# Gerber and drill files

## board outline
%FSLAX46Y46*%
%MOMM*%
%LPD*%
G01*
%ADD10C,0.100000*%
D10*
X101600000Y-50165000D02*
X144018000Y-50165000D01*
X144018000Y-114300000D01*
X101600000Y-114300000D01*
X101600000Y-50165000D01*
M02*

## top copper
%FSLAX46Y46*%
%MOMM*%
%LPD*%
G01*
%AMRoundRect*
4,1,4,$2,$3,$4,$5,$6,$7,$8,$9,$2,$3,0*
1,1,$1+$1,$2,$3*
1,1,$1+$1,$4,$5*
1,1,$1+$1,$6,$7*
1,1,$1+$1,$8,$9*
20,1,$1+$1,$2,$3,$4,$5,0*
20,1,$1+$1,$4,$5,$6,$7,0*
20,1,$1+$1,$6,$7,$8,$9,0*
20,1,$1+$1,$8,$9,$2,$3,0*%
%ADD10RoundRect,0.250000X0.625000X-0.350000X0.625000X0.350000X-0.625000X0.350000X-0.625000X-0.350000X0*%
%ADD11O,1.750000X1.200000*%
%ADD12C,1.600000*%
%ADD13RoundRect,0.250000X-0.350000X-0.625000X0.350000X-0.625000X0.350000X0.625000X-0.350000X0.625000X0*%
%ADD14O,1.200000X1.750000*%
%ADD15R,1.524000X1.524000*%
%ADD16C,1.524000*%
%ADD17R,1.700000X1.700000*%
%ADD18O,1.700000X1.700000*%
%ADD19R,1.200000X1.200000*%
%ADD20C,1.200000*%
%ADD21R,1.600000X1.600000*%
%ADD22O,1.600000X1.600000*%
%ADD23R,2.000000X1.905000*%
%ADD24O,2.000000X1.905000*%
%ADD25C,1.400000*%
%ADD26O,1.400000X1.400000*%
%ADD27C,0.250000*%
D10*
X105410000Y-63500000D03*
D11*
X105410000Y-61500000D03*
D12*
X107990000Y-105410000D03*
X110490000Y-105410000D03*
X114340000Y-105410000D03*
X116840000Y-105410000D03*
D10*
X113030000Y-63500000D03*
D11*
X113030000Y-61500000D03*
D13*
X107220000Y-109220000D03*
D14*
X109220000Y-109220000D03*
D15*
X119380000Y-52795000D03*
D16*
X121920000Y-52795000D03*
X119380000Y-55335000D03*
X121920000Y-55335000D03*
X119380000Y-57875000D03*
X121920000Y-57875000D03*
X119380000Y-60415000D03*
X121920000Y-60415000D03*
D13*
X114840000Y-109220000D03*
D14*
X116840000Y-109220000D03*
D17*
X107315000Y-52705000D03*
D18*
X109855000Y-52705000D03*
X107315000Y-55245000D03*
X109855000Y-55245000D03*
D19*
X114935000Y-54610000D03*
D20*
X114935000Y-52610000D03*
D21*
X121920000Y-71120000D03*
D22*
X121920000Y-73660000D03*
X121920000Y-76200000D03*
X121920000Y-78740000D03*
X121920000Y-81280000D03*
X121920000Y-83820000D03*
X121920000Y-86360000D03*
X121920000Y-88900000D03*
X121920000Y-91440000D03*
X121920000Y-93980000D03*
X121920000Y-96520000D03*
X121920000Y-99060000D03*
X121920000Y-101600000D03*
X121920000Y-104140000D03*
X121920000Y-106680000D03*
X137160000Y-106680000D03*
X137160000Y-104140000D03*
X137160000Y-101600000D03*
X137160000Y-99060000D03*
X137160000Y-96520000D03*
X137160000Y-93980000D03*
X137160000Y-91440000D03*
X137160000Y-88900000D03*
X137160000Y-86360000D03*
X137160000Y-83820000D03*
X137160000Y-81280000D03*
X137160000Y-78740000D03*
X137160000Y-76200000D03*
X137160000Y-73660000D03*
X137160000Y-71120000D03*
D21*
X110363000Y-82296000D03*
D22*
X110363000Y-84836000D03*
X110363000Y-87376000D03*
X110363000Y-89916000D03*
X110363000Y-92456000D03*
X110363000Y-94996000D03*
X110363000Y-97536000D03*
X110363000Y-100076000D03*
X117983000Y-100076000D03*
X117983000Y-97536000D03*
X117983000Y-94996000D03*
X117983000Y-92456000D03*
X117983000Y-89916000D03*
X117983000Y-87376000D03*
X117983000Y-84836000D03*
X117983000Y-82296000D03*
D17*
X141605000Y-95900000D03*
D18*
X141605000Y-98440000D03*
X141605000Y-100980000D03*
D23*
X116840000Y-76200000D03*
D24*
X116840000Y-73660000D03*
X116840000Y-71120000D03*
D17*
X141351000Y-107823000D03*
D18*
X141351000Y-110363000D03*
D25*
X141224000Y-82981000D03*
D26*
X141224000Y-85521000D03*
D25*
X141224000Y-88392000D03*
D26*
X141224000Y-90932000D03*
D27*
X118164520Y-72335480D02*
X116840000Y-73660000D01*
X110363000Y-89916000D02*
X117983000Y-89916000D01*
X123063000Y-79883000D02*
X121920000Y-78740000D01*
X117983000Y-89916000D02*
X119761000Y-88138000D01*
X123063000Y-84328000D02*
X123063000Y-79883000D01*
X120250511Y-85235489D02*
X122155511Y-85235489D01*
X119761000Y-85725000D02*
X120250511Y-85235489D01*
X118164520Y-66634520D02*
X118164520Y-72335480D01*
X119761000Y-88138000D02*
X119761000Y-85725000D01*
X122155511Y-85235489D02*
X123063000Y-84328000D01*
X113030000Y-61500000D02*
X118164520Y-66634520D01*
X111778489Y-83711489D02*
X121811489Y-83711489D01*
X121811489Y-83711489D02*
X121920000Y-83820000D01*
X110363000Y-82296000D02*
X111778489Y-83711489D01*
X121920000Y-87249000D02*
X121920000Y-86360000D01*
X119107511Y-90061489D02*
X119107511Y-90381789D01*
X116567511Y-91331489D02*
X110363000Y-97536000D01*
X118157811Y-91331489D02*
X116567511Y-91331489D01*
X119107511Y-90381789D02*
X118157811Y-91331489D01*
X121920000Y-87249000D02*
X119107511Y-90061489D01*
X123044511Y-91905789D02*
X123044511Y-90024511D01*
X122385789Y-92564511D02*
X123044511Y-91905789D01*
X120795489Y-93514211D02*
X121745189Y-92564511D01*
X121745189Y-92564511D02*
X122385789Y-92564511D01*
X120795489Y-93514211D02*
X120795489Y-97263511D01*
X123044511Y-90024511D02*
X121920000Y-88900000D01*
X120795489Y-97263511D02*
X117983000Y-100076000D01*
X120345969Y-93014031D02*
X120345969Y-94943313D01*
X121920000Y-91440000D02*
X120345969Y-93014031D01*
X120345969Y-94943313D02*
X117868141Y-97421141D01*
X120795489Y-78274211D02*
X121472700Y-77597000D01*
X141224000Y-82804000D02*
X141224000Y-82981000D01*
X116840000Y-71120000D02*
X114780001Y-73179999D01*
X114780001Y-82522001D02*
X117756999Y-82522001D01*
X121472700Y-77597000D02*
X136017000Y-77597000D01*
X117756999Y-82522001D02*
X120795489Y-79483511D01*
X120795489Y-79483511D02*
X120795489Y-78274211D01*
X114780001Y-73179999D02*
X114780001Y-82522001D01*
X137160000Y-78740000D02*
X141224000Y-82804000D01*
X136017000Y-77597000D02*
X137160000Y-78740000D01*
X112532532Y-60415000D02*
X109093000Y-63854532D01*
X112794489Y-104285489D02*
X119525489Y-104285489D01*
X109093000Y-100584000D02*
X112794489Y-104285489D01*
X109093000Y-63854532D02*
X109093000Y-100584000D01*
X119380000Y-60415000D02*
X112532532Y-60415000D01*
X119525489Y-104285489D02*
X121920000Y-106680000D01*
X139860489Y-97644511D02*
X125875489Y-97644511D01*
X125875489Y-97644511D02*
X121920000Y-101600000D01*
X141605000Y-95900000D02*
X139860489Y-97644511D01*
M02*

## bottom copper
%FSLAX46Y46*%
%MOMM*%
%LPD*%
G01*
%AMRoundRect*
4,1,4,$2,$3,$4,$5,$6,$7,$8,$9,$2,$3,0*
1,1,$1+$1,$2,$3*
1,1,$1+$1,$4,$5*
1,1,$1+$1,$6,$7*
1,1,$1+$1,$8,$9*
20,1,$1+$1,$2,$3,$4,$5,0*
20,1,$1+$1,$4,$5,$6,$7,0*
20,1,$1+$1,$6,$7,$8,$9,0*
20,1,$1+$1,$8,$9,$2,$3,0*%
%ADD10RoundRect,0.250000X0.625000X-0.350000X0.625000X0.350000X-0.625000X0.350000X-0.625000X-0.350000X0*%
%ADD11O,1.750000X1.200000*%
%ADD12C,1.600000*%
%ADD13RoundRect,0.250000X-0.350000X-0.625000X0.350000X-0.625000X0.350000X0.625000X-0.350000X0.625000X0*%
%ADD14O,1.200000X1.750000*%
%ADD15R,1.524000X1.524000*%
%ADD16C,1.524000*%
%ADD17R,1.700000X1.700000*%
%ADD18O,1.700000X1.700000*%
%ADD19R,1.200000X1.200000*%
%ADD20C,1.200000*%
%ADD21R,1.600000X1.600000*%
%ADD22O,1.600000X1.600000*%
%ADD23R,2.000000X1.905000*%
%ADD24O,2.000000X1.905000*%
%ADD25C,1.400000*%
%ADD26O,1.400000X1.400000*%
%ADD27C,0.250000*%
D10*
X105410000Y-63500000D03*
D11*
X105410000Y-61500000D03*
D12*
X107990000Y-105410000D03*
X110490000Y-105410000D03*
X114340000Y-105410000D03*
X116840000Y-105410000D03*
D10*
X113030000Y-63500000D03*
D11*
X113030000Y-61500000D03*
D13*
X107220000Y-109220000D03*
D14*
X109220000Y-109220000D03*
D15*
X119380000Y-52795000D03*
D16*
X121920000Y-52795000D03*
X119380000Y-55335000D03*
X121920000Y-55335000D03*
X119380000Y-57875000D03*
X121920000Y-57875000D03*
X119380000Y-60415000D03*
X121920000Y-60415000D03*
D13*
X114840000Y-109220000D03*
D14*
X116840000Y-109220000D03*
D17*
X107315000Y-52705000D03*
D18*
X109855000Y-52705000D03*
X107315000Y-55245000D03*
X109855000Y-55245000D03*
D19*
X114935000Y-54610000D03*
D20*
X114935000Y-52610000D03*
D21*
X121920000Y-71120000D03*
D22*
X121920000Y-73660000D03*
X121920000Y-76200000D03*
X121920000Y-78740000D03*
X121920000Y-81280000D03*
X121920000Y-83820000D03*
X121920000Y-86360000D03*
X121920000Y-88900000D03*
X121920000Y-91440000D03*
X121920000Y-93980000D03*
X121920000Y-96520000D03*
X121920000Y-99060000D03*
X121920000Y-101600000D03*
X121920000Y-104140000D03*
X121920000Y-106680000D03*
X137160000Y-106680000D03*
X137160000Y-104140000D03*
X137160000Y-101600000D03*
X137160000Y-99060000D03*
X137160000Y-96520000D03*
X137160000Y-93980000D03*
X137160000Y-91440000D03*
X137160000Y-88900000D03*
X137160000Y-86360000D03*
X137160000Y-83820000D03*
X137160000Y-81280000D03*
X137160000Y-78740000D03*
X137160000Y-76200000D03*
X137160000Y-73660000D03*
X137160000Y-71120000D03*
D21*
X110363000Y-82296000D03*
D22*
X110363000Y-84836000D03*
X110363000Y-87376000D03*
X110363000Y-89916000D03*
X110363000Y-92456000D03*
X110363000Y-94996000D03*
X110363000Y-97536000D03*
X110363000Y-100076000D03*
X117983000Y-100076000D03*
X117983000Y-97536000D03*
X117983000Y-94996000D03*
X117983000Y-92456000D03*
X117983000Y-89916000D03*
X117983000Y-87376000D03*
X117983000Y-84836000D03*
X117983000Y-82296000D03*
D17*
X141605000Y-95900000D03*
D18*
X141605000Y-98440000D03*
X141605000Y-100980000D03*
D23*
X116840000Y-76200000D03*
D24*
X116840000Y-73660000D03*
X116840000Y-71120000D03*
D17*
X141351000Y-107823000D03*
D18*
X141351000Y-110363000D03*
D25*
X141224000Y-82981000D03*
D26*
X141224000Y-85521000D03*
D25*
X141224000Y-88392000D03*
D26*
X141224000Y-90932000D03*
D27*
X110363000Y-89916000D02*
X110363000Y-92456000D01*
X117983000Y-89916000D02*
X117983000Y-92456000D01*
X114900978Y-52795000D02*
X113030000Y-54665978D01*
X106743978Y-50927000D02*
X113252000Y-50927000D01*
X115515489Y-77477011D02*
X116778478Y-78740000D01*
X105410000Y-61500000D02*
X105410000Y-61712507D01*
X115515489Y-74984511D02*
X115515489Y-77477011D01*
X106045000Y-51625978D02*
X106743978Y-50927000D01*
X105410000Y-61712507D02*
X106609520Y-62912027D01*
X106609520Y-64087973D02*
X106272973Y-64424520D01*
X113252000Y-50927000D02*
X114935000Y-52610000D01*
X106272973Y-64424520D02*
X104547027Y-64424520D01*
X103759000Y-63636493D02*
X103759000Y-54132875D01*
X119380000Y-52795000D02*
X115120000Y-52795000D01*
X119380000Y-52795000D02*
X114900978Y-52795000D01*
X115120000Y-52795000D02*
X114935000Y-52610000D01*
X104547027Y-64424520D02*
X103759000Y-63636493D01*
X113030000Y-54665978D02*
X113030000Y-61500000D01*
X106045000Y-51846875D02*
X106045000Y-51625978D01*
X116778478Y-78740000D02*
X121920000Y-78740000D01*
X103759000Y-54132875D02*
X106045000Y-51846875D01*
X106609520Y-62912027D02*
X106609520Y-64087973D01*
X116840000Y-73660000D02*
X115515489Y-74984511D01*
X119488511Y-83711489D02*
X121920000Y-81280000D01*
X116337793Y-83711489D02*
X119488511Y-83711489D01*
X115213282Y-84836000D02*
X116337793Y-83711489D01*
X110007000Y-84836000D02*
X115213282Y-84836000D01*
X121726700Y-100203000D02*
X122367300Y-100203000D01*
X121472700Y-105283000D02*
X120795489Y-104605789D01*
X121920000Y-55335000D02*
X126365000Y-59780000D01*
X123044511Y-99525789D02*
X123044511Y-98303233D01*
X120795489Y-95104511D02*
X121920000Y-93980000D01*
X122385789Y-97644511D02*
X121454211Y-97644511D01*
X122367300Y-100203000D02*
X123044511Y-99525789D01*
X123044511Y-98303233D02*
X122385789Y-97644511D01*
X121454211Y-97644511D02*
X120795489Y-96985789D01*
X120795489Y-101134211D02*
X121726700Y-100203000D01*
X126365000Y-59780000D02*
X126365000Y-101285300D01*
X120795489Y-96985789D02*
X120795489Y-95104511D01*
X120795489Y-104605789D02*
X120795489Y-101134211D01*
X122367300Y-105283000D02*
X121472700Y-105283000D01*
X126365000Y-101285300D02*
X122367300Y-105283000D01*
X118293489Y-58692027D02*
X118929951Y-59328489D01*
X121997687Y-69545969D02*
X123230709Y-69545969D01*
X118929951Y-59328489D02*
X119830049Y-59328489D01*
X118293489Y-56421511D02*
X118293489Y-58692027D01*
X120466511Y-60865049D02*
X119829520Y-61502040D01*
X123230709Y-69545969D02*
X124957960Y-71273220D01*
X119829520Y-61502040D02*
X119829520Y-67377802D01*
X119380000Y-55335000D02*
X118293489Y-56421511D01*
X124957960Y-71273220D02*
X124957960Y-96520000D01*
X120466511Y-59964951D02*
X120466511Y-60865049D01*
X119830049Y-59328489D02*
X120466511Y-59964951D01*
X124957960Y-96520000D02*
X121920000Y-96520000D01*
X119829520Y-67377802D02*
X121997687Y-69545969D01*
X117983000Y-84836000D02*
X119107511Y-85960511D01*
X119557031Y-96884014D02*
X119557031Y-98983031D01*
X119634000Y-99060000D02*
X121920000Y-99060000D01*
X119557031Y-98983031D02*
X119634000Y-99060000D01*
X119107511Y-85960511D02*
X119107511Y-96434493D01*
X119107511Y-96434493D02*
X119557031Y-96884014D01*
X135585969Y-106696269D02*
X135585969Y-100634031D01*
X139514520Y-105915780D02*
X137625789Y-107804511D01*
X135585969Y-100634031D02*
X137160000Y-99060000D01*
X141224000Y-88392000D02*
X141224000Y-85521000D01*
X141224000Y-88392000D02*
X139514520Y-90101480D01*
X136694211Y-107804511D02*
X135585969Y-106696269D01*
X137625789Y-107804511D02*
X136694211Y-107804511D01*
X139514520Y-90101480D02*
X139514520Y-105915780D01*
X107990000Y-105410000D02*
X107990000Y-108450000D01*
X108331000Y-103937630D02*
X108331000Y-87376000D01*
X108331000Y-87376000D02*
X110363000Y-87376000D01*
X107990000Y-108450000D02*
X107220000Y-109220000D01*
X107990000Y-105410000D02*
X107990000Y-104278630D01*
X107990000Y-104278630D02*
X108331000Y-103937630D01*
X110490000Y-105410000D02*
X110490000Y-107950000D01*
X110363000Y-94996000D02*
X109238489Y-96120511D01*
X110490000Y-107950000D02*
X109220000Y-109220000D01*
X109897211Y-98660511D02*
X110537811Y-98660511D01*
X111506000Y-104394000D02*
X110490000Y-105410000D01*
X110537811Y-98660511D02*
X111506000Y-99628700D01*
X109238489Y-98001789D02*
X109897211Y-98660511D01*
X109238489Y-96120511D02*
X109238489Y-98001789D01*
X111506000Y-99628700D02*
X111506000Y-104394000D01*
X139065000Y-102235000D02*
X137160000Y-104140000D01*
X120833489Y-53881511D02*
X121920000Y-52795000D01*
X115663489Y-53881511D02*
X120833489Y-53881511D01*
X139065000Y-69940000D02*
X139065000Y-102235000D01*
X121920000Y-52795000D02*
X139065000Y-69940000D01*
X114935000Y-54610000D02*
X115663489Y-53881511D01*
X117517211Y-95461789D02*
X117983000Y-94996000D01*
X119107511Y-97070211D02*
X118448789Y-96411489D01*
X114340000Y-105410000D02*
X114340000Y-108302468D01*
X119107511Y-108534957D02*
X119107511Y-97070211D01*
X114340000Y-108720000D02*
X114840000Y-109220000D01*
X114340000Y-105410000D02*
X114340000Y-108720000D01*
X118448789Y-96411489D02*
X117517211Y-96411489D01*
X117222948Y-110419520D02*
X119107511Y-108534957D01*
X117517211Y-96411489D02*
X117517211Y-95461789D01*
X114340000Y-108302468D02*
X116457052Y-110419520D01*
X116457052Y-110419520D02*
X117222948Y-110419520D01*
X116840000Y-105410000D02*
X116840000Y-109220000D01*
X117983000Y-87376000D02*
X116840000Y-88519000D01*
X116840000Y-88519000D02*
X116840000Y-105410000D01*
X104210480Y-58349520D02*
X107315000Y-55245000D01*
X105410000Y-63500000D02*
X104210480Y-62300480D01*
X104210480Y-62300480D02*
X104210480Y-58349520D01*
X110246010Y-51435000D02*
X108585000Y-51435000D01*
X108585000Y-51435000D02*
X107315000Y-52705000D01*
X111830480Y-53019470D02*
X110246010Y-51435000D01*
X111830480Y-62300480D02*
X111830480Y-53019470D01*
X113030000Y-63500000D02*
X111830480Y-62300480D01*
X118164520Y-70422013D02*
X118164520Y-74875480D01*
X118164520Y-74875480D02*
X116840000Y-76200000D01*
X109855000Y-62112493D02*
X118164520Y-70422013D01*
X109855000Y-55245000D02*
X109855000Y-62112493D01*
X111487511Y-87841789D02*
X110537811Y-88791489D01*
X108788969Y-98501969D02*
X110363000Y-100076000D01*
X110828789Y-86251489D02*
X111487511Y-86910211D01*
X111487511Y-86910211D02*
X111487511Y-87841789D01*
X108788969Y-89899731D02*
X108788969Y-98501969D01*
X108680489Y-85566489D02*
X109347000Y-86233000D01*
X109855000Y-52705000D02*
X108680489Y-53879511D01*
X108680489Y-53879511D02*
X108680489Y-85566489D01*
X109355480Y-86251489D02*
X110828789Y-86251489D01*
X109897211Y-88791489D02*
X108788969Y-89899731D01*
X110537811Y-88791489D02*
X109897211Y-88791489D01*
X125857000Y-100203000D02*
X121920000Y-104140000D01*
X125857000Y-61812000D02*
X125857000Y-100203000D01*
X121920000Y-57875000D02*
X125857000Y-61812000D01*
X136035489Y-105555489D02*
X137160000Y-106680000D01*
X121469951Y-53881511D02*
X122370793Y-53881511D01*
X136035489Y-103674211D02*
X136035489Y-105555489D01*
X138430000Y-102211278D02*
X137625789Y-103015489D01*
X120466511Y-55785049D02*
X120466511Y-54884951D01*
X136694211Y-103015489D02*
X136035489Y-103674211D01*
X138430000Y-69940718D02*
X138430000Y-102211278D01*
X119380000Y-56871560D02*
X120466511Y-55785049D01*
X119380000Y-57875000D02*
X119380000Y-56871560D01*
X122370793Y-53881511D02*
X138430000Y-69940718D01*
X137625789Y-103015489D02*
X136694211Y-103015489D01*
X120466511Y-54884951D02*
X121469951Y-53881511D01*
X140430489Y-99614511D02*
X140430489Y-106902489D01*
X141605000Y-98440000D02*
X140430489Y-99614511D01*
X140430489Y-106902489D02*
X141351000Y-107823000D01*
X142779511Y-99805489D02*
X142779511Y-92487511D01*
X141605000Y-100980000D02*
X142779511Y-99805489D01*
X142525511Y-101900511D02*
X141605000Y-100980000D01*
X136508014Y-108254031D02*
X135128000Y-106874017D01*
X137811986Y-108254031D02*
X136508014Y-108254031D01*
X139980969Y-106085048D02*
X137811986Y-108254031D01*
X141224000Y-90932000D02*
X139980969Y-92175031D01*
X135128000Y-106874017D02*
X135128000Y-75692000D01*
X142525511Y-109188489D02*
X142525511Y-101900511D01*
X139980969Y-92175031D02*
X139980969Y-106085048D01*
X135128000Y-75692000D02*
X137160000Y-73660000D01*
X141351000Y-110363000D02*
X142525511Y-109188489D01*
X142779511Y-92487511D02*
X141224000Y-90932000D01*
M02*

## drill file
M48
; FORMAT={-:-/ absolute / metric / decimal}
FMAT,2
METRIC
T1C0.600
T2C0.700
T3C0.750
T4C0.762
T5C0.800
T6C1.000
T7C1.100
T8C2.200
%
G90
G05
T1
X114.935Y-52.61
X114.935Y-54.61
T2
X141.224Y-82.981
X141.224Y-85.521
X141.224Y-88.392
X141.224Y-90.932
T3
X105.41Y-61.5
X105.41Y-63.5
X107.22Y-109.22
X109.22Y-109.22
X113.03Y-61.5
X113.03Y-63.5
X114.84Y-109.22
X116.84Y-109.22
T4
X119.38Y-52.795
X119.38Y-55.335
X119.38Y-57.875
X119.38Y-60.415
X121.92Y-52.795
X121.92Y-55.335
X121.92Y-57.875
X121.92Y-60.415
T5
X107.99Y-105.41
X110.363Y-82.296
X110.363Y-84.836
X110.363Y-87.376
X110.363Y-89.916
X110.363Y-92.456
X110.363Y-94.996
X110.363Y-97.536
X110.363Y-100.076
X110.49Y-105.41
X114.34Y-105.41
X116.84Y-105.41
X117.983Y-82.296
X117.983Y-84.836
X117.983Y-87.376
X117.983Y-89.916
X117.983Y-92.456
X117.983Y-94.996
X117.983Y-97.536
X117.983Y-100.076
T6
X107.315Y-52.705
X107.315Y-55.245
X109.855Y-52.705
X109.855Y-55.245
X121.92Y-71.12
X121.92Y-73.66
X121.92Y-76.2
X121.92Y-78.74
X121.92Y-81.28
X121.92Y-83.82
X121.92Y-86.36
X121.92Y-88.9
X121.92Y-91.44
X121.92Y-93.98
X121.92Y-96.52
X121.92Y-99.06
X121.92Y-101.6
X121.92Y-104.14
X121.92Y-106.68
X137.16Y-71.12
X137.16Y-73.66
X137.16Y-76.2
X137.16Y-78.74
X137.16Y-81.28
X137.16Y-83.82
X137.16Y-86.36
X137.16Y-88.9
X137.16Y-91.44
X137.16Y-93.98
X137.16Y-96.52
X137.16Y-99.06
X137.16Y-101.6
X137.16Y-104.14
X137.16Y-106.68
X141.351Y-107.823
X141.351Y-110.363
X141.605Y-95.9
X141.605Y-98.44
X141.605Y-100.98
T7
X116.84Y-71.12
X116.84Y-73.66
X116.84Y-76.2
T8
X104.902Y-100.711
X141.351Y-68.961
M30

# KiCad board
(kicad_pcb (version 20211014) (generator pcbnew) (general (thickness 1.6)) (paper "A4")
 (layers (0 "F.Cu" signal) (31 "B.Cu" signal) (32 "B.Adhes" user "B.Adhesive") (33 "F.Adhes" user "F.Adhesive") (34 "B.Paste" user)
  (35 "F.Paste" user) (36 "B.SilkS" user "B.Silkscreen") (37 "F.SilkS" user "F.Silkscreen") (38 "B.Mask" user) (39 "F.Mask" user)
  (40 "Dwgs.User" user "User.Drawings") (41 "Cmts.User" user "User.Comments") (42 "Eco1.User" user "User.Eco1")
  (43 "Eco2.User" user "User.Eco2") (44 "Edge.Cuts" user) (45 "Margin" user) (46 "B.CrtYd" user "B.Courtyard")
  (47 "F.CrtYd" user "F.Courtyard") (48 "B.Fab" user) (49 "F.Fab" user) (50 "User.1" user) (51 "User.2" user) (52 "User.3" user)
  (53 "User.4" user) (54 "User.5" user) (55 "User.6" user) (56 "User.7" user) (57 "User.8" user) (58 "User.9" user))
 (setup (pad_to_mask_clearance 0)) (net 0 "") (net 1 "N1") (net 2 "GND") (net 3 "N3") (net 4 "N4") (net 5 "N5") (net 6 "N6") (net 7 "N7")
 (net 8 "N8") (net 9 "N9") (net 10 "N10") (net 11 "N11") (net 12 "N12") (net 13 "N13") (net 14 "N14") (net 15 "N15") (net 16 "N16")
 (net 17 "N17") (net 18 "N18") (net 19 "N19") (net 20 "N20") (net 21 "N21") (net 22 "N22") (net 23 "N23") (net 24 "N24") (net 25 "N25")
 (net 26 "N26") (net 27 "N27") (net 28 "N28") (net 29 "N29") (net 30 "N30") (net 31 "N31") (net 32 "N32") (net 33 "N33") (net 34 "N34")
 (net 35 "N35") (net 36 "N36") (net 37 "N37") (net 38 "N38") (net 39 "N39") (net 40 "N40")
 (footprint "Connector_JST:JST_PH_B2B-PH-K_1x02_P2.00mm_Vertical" (layer "F.Cu") (at 105.41 63.5 90)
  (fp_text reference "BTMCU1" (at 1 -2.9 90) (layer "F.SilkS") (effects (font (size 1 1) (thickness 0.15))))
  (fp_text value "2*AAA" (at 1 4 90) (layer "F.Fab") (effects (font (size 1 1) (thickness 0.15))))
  (pad "1" thru_hole roundrect (at 0 0 90) (size 1.2 1.75) (drill 0.75) (layers *.Cu *.Mask) (roundrect_rratio 0.2083333333) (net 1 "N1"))
  (pad "2" thru_hole oval (at 2 0 90) (size 1.2 1.75) (drill 0.75) (layers *.Cu *.Mask) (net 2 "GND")))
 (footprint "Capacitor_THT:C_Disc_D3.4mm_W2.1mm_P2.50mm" (layer "F.Cu") (at 107.99 105.41)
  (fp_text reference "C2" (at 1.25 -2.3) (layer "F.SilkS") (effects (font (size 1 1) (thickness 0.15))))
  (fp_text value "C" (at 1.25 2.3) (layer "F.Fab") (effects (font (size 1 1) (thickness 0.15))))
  (pad "1" thru_hole circle (at 0 0) (size 1.6 1.6) (drill 0.8) (layers *.Cu *.Mask) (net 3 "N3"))
  (pad "2" thru_hole circle (at 2.5 0) (size 1.6 1.6) (drill 0.8) (layers *.Cu *.Mask) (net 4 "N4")))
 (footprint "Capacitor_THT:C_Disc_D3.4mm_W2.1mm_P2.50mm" (layer "F.Cu") (at 114.34 105.41)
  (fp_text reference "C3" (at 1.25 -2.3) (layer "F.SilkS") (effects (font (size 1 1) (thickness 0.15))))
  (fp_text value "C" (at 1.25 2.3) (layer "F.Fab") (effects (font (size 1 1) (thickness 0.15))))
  (pad "1" thru_hole circle (at 0 0) (size 1.6 1.6) (drill 0.8) (layers *.Cu *.Mask) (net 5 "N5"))
  (pad "2" thru_hole circle (at 2.5 0) (size 1.6 1.6) (drill 0.8) (layers *.Cu *.Mask) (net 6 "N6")))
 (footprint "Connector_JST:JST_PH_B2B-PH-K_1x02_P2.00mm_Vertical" (layer "F.Cu") (at 113.03 63.5 90)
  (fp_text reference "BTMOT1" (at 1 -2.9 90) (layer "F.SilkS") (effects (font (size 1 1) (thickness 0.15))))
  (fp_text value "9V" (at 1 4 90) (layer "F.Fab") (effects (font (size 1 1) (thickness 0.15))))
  (pad "1" thru_hole roundrect (at 0 0 90) (size 1.2 1.75) (drill 0.75) (layers *.Cu *.Mask) (roundrect_rratio 0.2083333333) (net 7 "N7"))
  (pad "2" thru_hole oval (at 2 0 90) (size 1.2 1.75) (drill 0.75) (layers *.Cu *.Mask) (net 2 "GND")))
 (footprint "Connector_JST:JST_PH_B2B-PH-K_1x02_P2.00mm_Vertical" (layer "F.Cu") (at 107.22 109.22)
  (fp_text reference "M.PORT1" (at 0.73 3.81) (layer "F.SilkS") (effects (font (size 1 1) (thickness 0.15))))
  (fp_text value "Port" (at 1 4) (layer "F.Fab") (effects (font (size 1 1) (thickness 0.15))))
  (pad "1" thru_hole roundrect (at 0 0) (size 1.2 1.75) (drill 0.75) (layers *.Cu *.Mask) (roundrect_rratio 0.2083333333) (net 3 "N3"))
  (pad "2" thru_hole oval (at 2 0) (size 1.2 1.75) (drill 0.75) (layers *.Cu *.Mask) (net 4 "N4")))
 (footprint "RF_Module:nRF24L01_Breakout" (layer "F.Cu") (at 119.38 52.795)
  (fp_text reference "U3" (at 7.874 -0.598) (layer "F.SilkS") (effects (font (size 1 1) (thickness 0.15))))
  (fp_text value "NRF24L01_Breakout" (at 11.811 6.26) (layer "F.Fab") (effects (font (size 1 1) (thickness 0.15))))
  (pad "1" thru_hole rect (at 0 0) (size 1.524 1.524) (drill 0.762) (layers *.Cu *.Mask) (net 2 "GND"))
  (pad "2" thru_hole circle (at 2.54 0) (size 1.524 1.524) (drill 0.762) (layers *.Cu *.Mask) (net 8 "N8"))
  (pad "3" thru_hole circle (at 0 2.54) (size 1.524 1.524) (drill 0.762) (layers *.Cu *.Mask) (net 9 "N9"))
  (pad "4" thru_hole circle (at 2.54 2.54) (size 1.524 1.524) (drill 0.762) (layers *.Cu *.Mask) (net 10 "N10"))
  (pad "5" thru_hole circle (at 0 5.08) (size 1.524 1.524) (drill 0.762) (layers *.Cu *.Mask) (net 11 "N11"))
  (pad "6" thru_hole circle (at 2.54 5.08) (size 1.524 1.524) (drill 0.762) (layers *.Cu *.Mask) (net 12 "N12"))
  (pad "7" thru_hole circle (at 0 7.62) (size 1.524 1.524) (drill 0.762) (layers *.Cu *.Mask) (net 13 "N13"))
  (pad "8" thru_hole circle (at 2.54 7.62) (size 1.524 1.524) (drill 0.762) (layers *.Cu *.Mask) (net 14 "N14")))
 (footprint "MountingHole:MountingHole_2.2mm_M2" (layer "F.Cu") (at 104.902 100.711)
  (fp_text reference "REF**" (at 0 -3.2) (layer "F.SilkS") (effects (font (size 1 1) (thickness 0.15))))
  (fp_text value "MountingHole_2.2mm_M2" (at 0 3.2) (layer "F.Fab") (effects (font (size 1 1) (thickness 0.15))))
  (pad "" np_thru_hole circle (at 0 0) (size 2.2 2.2) (drill 2.2) (layers *.Cu *.Mask)))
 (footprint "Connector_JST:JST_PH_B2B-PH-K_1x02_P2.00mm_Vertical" (layer "F.Cu") (at 114.84 109.22)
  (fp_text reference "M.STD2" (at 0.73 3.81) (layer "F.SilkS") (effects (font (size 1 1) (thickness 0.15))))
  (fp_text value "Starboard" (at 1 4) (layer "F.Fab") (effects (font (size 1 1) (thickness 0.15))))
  (pad "1" thru_hole roundrect (at 0 0) (size 1.2 1.75) (drill 0.75) (layers *.Cu *.Mask) (roundrect_rratio 0.2083333333) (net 5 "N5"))
  (pad "2" thru_hole oval (at 2 0) (size 1.2 1.75) (drill 0.75) (layers *.Cu *.Mask) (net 6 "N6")))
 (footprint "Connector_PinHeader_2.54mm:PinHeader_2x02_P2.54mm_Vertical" (layer "F.Cu") (at 107.315 52.705)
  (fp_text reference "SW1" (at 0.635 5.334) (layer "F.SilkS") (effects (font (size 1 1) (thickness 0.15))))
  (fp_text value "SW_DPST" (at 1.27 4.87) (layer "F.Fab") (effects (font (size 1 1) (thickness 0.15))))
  (pad "1" thru_hole rect (at 0 0) (size 1.7 1.7) (drill 1) (layers *.Cu *.Mask) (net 7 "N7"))
  (pad "2" thru_hole oval (at 2.54 0) (size 1.7 1.7) (drill 1) (layers *.Cu *.Mask) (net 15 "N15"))
  (pad "3" thru_hole oval (at 0 2.54) (size 1.7 1.7) (drill 1) (layers *.Cu *.Mask) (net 1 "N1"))
  (pad "4" thru_hole oval (at 2.54 2.54) (size 1.7 1.7) (drill 1) (layers *.Cu *.Mask) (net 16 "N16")))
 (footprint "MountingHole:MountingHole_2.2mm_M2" (layer "F.Cu") (at 141.351 68.961)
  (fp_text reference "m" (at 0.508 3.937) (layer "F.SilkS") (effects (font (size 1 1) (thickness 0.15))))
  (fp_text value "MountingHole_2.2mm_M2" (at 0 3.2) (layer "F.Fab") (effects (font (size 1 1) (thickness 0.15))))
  (pad "" np_thru_hole circle (at 0 0) (size 2.2 2.2) (drill 2.2) (layers *.Cu *.Mask)))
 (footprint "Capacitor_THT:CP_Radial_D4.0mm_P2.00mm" (layer "F.Cu") (at 114.935 54.61 90)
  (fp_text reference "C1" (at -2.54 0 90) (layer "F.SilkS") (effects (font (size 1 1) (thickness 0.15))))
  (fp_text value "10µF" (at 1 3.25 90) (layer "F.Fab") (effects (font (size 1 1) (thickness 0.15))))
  (pad "1" thru_hole rect (at 0 0 90) (size 1.2 1.2) (drill 0.6) (layers *.Cu *.Mask) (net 8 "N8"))
  (pad "2" thru_hole circle (at 2 0 90) (size 1.2 1.2) (drill 0.6) (layers *.Cu *.Mask) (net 2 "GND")))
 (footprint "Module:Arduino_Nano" (layer "F.Cu") (at 121.92 71.12)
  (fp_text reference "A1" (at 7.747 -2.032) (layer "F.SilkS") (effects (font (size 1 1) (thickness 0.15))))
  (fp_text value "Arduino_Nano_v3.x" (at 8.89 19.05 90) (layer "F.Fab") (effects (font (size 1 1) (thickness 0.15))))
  (pad "1" thru_hole rect (at 0 0) (size 1.6 1.6) (drill 1) (layers *.Cu *.Mask) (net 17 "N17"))
  (pad "2" thru_hole oval (at 0 2.54) (size 1.6 1.6) (drill 1) (layers *.Cu *.Mask) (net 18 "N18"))
  (pad "3" thru_hole oval (at 0 5.08) (size 1.6 1.6) (drill 1) (layers *.Cu *.Mask) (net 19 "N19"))
  (pad "4" thru_hole oval (at 0 7.62) (size 1.6 1.6) (drill 1) (layers *.Cu *.Mask) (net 2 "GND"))
  (pad "5" thru_hole oval (at 0 10.16) (size 1.6 1.6) (drill 1) (layers *.Cu *.Mask) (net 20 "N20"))
  (pad "6" thru_hole oval (at 0 12.7) (size 1.6 1.6) (drill 1) (layers *.Cu *.Mask) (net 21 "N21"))
  (pad "7" thru_hole oval (at 0 15.24) (size 1.6 1.6) (drill 1) (layers *.Cu *.Mask) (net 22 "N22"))
  (pad "8" thru_hole oval (at 0 17.78) (size 1.6 1.6) (drill 1) (layers *.Cu *.Mask) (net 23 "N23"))
  (pad "9" thru_hole oval (at 0 20.32) (size 1.6 1.6) (drill 1) (layers *.Cu *.Mask) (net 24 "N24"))
  (pad "10" thru_hole oval (at 0 22.86) (size 1.6 1.6) (drill 1) (layers *.Cu *.Mask) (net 10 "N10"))
  (pad "11" thru_hole oval (at 0 25.4) (size 1.6 1.6) (drill 1) (layers *.Cu *.Mask) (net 9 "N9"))
  (pad "12" thru_hole oval (at 0 27.94) (size 1.6 1.6) (drill 1) (layers *.Cu *.Mask) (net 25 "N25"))
  (pad "13" thru_hole oval (at 0 30.48) (size 1.6 1.6) (drill 1) (layers *.Cu *.Mask) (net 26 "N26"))
  (pad "14" thru_hole oval (at 0 33.02) (size 1.6 1.6) (drill 1) (layers *.Cu *.Mask) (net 12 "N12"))
  (pad "15" thru_hole oval (at 0 35.56) (size 1.6 1.6) (drill 1) (layers *.Cu *.Mask) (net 13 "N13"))
  (pad "16" thru_hole oval (at 15.24 35.56) (size 1.6 1.6) (drill 1) (layers *.Cu *.Mask) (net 11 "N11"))
  (pad "17" thru_hole oval (at 15.24 33.02) (size 1.6 1.6) (drill 1) (layers *.Cu *.Mask) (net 8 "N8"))
  (pad "18" thru_hole oval (at 15.24 30.48) (size 1.6 1.6) (drill 1) (layers *.Cu *.Mask) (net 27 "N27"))
  (pad "19" thru_hole oval (at 15.24 27.94) (size 1.6 1.6) (drill 1) (layers *.Cu *.Mask) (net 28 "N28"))
  (pad "20" thru_hole oval (at 15.24 25.4) (size 1.6 1.6) (drill 1) (layers *.Cu *.Mask) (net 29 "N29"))
  (pad "21" thru_hole oval (at 15.24 22.86) (size 1.6 1.6) (drill 1) (layers *.Cu *.Mask) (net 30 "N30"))
  (pad "22" thru_hole oval (at 15.24 20.32) (size 1.6 1.6) (drill 1) (layers *.Cu *.Mask) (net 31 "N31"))
  (pad "23" thru_hole oval (at 15.24 17.78) (size 1.6 1.6) (drill 1) (layers *.Cu *.Mask) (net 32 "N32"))
  (pad "24" thru_hole oval (at 15.24 15.24) (size 1.6 1.6) (drill 1) (layers *.Cu *.Mask) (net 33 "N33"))
  (pad "25" thru_hole oval (at 15.24 12.7) (size 1.6 1.6) (drill 1) (layers *.Cu *.Mask) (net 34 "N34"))
  (pad "26" thru_hole oval (at 15.24 10.16) (size 1.6 1.6) (drill 1) (layers *.Cu *.Mask) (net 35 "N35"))
  (pad "27" thru_hole oval (at 15.24 7.62) (size 1.6 1.6) (drill 1) (layers *.Cu *.Mask) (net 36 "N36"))
  (pad "28" thru_hole oval (at 15.24 5.08) (size 1.6 1.6) (drill 1) (layers *.Cu *.Mask) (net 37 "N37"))
  (pad "29" thru_hole oval (at 15.24 2.54) (size 1.6 1.6) (drill 1) (layers *.Cu *.Mask) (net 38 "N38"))
  (pad "30" thru_hole oval (at 15.24 0) (size 1.6 1.6) (drill 1) (layers *.Cu *.Mask) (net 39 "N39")))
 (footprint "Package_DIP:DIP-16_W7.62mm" (layer "F.Cu") (at 110.363 82.296)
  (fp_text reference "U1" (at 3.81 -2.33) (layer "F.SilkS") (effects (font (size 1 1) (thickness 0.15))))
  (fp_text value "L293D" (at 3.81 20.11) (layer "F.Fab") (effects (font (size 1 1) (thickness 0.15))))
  (pad "1" thru_hole rect (at 0 0) (size 1.6 1.6) (drill 0.8) (layers *.Cu *.Mask) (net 21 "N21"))
  (pad "2" thru_hole oval (at 0 2.54) (size 1.6 1.6) (drill 0.8) (layers *.Cu *.Mask) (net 20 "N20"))
  (pad "3" thru_hole oval (at 0 5.08) (size 1.6 1.6) (drill 0.8) (layers *.Cu *.Mask) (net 3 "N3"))
  (pad "4" thru_hole oval (at 0 7.62) (size 1.6 1.6) (drill 0.8) (layers *.Cu *.Mask) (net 2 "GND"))
  (pad "5" thru_hole oval (at 0 10.16) (size 1.6 1.6) (drill 0.8) (layers *.Cu *.Mask) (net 2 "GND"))
  (pad "6" thru_hole oval (at 0 12.7) (size 1.6 1.6) (drill 0.8) (layers *.Cu *.Mask) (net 4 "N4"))
  (pad "7" thru_hole oval (at 0 15.24) (size 1.6 1.6) (drill 0.8) (layers *.Cu *.Mask) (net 22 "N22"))
  (pad "8" thru_hole oval (at 0 17.78) (size 1.6 1.6) (drill 0.8) (layers *.Cu *.Mask) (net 15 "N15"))
  (pad "9" thru_hole oval (at 7.62 17.78) (size 1.6 1.6) (drill 0.8) (layers *.Cu *.Mask) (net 23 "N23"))
  (pad "10" thru_hole oval (at 7.62 15.24) (size 1.6 1.6) (drill 0.8) (layers *.Cu *.Mask) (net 24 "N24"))
  (pad "11" thru_hole oval (at 7.62 12.7) (size 1.6 1.6) (drill 0.8) (layers *.Cu *.Mask) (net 5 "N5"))
  (pad "12" thru_hole oval (at 7.62 10.16) (size 1.6 1.6) (drill 0.8) (layers *.Cu *.Mask) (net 2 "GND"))
  (pad "13" thru_hole oval (at 7.62 7.62) (size 1.6 1.6) (drill 0.8) (layers *.Cu *.Mask) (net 2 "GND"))
  (pad "14" thru_hole oval (at 7.62 5.08) (size 1.6 1.6) (drill 0.8) (layers *.Cu *.Mask) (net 6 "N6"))
  (pad "15" thru_hole oval (at 7.62 2.54) (size 1.6 1.6) (drill 0.8) (layers *.Cu *.Mask) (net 25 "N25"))
  (pad "16" thru_hole oval (at 7.62 0) (size 1.6 1.6) (drill 0.8) (layers *.Cu *.Mask) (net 36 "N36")))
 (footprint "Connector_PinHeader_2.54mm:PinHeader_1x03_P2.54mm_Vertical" (layer "F.Cu") (at 141.605 95.9)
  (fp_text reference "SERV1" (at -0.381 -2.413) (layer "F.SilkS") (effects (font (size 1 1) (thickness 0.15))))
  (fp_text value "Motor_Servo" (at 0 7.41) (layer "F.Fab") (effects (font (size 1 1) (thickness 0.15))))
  (pad "1" thru_hole rect (at 0 0) (size 1.7 1.7) (drill 1) (layers *.Cu *.Mask) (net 26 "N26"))
  (pad "2" thru_hole oval (at 0 2.54) (size 1.7 1.7) (drill 1) (layers *.Cu *.Mask) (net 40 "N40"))
  (pad "3" thru_hole oval (at 0 5.08) (size 1.7 1.7) (drill 1) (layers *.Cu *.Mask) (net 38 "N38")))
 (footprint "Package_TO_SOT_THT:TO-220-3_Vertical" (layer "F.Cu") (at 116.84 76.2 90)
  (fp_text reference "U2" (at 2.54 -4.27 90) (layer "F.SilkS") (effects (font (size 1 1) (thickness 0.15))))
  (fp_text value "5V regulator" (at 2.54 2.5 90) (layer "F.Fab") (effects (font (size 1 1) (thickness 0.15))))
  (pad "1" thru_hole rect (at 0 0 90) (size 1.905 2) (drill 1.1) (layers *.Cu *.Mask) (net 16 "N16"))
  (pad "2" thru_hole oval (at 2.54 0 90) (size 1.905 2) (drill 1.1) (layers *.Cu *.Mask) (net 2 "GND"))
  (pad "3" thru_hole oval (at 5.08 0 90) (size 1.905 2) (drill 1.1) (layers *.Cu *.Mask) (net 36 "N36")))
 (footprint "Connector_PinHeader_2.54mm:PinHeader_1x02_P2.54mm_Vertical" (layer "F.Cu") (at 141.351 107.823)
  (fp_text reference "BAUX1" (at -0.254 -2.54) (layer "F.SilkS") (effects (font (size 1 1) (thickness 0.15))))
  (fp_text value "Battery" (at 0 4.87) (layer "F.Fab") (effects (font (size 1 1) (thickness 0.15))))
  (pad "1" thru_hole rect (at 0 0) (size 1.7 1.7) (drill 1) (layers *.Cu *.Mask) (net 40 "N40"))
  (pad "2" thru_hole oval (at 0 2.54) (size 1.7 1.7) (drill 1) (layers *.Cu *.Mask) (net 38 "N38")))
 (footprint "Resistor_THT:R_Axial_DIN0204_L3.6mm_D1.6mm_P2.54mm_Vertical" (layer "F.Cu") (at 141.224 82.981 -90)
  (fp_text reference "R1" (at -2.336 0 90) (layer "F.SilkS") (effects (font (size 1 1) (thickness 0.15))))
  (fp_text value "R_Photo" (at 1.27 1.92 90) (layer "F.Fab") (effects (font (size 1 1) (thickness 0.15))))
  (pad "1" thru_hole circle (at 0 0 270) (size 1.4 1.4) (drill 0.7) (layers *.Cu *.Mask) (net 36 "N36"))
  (pad "2" thru_hole oval (at 2.54 0 270) (size 1.4 1.4) (drill 0.7) (layers *.Cu *.Mask) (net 28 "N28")))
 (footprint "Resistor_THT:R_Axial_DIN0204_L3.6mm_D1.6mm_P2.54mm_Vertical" (layer "F.Cu") (at 141.224 88.392 -90)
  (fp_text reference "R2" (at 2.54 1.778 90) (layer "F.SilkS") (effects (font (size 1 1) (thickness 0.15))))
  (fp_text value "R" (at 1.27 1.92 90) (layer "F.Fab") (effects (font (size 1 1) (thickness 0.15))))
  (pad "1" thru_hole circle (at 0 0 270) (size 1.4 1.4) (drill 0.7) (layers *.Cu *.Mask) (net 28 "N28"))
  (pad "2" thru_hole oval (at 2.54 0 270) (size 1.4 1.4) (drill 0.7) (layers *.Cu *.Mask) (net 38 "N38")))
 (gr_rect (start 144.018 50.165) (end 101.6 114.3) (layer "Edge.Cuts") (width 0.1) (fill none))
 (segment (start 118.16452 72.33548) (end 116.84 73.66) (width 0.25) (layer "F.Cu") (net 2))
 (segment (start 110.363 89.916) (end 117.983 89.916) (width 0.25) (layer "F.Cu") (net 2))
 (segment (start 123.063 79.883) (end 121.92 78.74) (width 0.25) (layer "F.Cu") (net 2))
 (segment (start 117.983 89.916) (end 119.761 88.138) (width 0.25) (layer "F.Cu") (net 2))
 (segment (start 123.063 84.328) (end 123.063 79.883) (width 0.25) (layer "F.Cu") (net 2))
 (segment (start 120.250511 85.235489) (end 122.155511 85.235489) (width 0.25) (layer "F.Cu") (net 2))
 (segment (start 119.761 85.725) (end 120.250511 85.235489) (width 0.25) (layer "F.Cu") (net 2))
 (segment (start 118.16452 66.63452) (end 118.16452 72.33548) (width 0.25) (layer "F.Cu") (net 2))
 (segment (start 119.761 88.138) (end 119.761 85.725) (width 0.25) (layer "F.Cu") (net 2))
 (segment (start 122.155511 85.235489) (end 123.063 84.328) (width 0.25) (layer "F.Cu") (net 2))
 (segment (start 113.03 61.5) (end 118.16452 66.63452) (width 0.25) (layer "F.Cu") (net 2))
 (segment (start 110.363 89.916) (end 110.363 92.456) (width 0.25) (layer "B.Cu") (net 2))
 (segment (start 117.983 89.916) (end 117.983 92.456) (width 0.25) (layer "B.Cu") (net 2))
 (segment (start 114.900978 52.795) (end 113.03 54.665978) (width 0.25) (layer "B.Cu") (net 2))
 (segment (start 106.743978 50.927) (end 113.252 50.927) (width 0.25) (layer "B.Cu") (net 2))
 (segment (start 115.515489 77.477011) (end 116.778478 78.74) (width 0.25) (layer "B.Cu") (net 2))
 (segment (start 105.41 61.5) (end 105.41 61.712507) (width 0.25) (layer "B.Cu") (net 2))
 (segment (start 115.515489 74.984511) (end 115.515489 77.477011) (width 0.25) (layer "B.Cu") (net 2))
 (segment (start 106.045 51.625978) (end 106.743978 50.927) (width 0.25) (layer "B.Cu") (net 2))
 (segment (start 105.41 61.712507) (end 106.60952 62.912027) (width 0.25) (layer "B.Cu") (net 2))
 (segment (start 106.60952 64.087973) (end 106.272973 64.42452) (width 0.25) (layer "B.Cu") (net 2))
 (segment (start 113.252 50.927) (end 114.935 52.61) (width 0.25) (layer "B.Cu") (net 2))
 (segment (start 106.272973 64.42452) (end 104.547027 64.42452) (width 0.25) (layer "B.Cu") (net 2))
 (segment (start 103.759 63.636493) (end 103.759 54.132875) (width 0.25) (layer "B.Cu") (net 2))
 (segment (start 119.38 52.795) (end 115.12 52.795) (width 0.25) (layer "B.Cu") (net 2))
 (segment (start 119.38 52.795) (end 114.900978 52.795) (width 0.25) (layer "B.Cu") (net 2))
 (segment (start 115.12 52.795) (end 114.935 52.61) (width 0.25) (layer "B.Cu") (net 2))
 (segment (start 104.547027 64.42452) (end 103.759 63.636493) (width 0.25) (layer "B.Cu") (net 2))
 (segment (start 113.03 54.665978) (end 113.03 61.5) (width 0.25) (layer "B.Cu") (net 2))
 (segment (start 106.045 51.846875) (end 106.045 51.625978) (width 0.25) (layer "B.Cu") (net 2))
 (segment (start 116.778478 78.74) (end 121.92 78.74) (width 0.25) (layer "B.Cu") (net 2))
 (segment (start 103.759 54.132875) (end 106.045 51.846875) (width 0.25) (layer "B.Cu") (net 2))
 (segment (start 106.60952 62.912027) (end 106.60952 64.087973) (width 0.25) (layer "B.Cu") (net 2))
 (segment (start 116.84 73.66) (end 115.515489 74.984511) (width 0.25) (layer "B.Cu") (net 2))
 (segment (start 119.488511 83.711489) (end 121.92 81.28) (width 0.25) (layer "B.Cu") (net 20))
 (segment (start 116.337793 83.711489) (end 119.488511 83.711489) (width 0.25) (layer "B.Cu") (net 20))
 (segment (start 115.213282 84.836) (end 116.337793 83.711489) (width 0.25) (layer "B.Cu") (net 20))
 (segment (start 110.007 84.836) (end 115.213282 84.836) (width 0.25) (layer "B.Cu") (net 20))
 (segment (start 111.778489 83.711489) (end 121.811489 83.711489) (width 0.25) (layer "F.Cu") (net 21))
 (segment (start 121.811489 83.711489) (end 121.92 83.82) (width 0.25) (layer "F.Cu") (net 21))
 (segment (start 110.363 82.296) (end 111.778489 83.711489) (width 0.25) (layer "F.Cu") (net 21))
 (segment (start 121.92 87.249) (end 121.92 86.36) (width 0.25) (layer "F.Cu") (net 22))
 (segment (start 119.107511 90.061489) (end 119.107511 90.381789) (width 0.25) (layer "F.Cu") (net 22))
 (segment (start 116.567511 91.331489) (end 110.363 97.536) (width 0.25) (layer "F.Cu") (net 22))
 (segment (start 118.157811 91.331489) (end 116.567511 91.331489) (width 0.25) (layer "F.Cu") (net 22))
 (segment (start 119.107511 90.381789) (end 118.157811 91.331489) (width 0.25) (layer "F.Cu") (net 22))
 (segment (start 121.92 87.249) (end 119.107511 90.061489) (width 0.25) (layer "F.Cu") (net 22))
 (segment (start 123.044511 91.905789) (end 123.044511 90.024511) (width 0.25) (layer "F.Cu") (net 23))
 (segment (start 122.385789 92.564511) (end 123.044511 91.905789) (width 0.25) (layer "F.Cu") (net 23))
 (segment (start 120.795489 93.514211) (end 121.745189 92.564511) (width 0.25) (layer "F.Cu") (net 23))
 (segment (start 121.745189 92.564511) (end 122.385789 92.564511) (width 0.25) (layer "F.Cu") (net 23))
 (segment (start 120.795489 93.514211) (end 120.795489 97.263511) (width 0.25) (layer "F.Cu") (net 23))
 (segment (start 123.044511 90.024511) (end 121.92 88.9) (width 0.25) (layer "F.Cu") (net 23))
 (segment (start 120.795489 97.263511) (end 117.983 100.076) (width 0.25) (layer "F.Cu") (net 23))
 (segment (start 120.345969 93.014031) (end 120.345969 94.943313) (width 0.25) (layer "F.Cu") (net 24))
 (segment (start 121.92 91.44) (end 120.345969 93.014031) (width 0.25) (layer "F.Cu") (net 24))
 (segment (start 120.345969 94.943313) (end 117.868141 97.421141) (width 0.25) (layer "F.Cu") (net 24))
 (segment (start 121.7267 100.203) (end 122.3673 100.203) (width 0.25) (layer "B.Cu") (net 10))
 (segment (start 121.4727 105.283) (end 120.795489 104.605789) (width 0.25) (layer "B.Cu") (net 10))
 (segment (start 121.92 55.335) (end 126.365 59.78) (width 0.25) (layer "B.Cu") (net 10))
 (segment (start 123.044511 99.525789) (end 123.044511 98.303233) (width 0.25) (layer "B.Cu") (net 10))
 (segment (start 120.795489 95.104511) (end 121.92 93.98) (width 0.25) (layer "B.Cu") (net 10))
 (segment (start 122.385789 97.644511) (end 121.454211 97.644511) (width 0.25) (layer "B.Cu") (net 10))
 (segment (start 122.3673 100.203) (end 123.044511 99.525789) (width 0.25) (layer "B.Cu") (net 10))
 (segment (start 123.044511 98.303233) (end 122.385789 97.644511) (width 0.25) (layer "B.Cu") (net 10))
 (segment (start 121.454211 97.644511) (end 120.795489 96.985789) (width 0.25) (layer "B.Cu") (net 10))
 (segment (start 120.795489 101.134211) (end 121.7267 100.203) (width 0.25) (layer "B.Cu") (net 10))
 (segment (start 126.365 59.78) (end 126.365 101.2853) (width 0.25) (layer "B.Cu") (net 10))
 (segment (start 120.795489 96.985789) (end 120.795489 95.104511) (width 0.25) (layer "B.Cu") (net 10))
 (segment (start 120.795489 104.605789) (end 120.795489 101.134211) (width 0.25) (layer "B.Cu") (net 10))
 (segment (start 122.3673 105.283) (end 121.4727 105.283) (width 0.25) (layer "B.Cu") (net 10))
 (segment (start 126.365 101.2853) (end 122.3673 105.283) (width 0.25) (layer "B.Cu") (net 10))
 (segment (start 118.293489 58.692027) (end 118.929951 59.328489) (width 0.25) (layer "B.Cu") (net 9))
 (segment (start 121.997687 69.545969) (end 123.230709 69.545969) (width 0.25) (layer "B.Cu") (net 9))
 (segment (start 118.929951 59.328489) (end 119.830049 59.328489) (width 0.25) (layer "B.Cu") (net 9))
 (segment (start 118.293489 56.421511) (end 118.293489 58.692027) (width 0.25) (layer "B.Cu") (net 9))
 (segment (start 120.466511 60.865049) (end 119.82952 61.50204) (width 0.25) (layer "B.Cu") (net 9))
 (segment (start 123.230709 69.545969) (end 124.95796 71.27322) (width 0.25) (layer "B.Cu") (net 9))
 (segment (start 119.82952 61.50204) (end 119.82952 67.377802) (width 0.25) (layer "B.Cu") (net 9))
 (segment (start 119.38 55.335) (end 118.293489 56.421511) (width 0.25) (layer "B.Cu") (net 9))
 (segment (start 124.95796 71.27322) (end 124.95796 96.52) (width 0.25) (layer "B.Cu") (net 9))
 (segment (start 120.466511 59.964951) (end 120.466511 60.865049) (width 0.25) (layer "B.Cu") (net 9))
 (segment (start 119.830049 59.328489) (end 120.466511 59.964951) (width 0.25) (layer "B.Cu") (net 9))
 (segment (start 124.95796 96.52) (end 121.92 96.52) (width 0.25) (layer "B.Cu") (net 9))
 (segment (start 119.82952 67.377802) (end 121.997687 69.545969) (width 0.25) (layer "B.Cu") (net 9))
 (segment (start 117.983 84.836) (end 119.107511 85.960511) (width 0.25) (layer "B.Cu") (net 25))
 (segment (start 119.557031 96.884014) (end 119.557031 98.983031) (width 0.25) (layer "B.Cu") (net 25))
 (segment (start 119.634 99.06) (end 121.92 99.06) (width 0.25) (layer "B.Cu") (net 25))
 (segment (start 119.557031 98.983031) (end 119.634 99.06) (width 0.25) (layer "B.Cu") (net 25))
 (segment (start 119.107511 85.960511) (end 119.107511 96.434493) (width 0.25) (layer "B.Cu") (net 25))
 (segment (start 119.107511 96.434493) (end 119.557031 96.884014) (width 0.25) (layer "B.Cu") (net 25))
 (segment (start 135.585969 106.696269) (end 135.585969 100.634031) (width 0.25) (layer "B.Cu") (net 28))
 (segment (start 139.51452 105.91578) (end 137.625789 107.804511) (width 0.25) (layer "B.Cu") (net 28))
 (segment (start 135.585969 100.634031) (end 137.16 99.06) (width 0.25) (layer "B.Cu") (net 28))
 (segment (start 141.224 88.392) (end 141.224 85.521) (width 0.25) (layer "B.Cu") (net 28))
 (segment (start 141.224 88.392) (end 139.51452 90.10148) (width 0.25) (layer "B.Cu") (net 28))
 (segment (start 136.694211 107.804511) (end 135.585969 106.696269) (width 0.25) (layer "B.Cu") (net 28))
 (segment (start 137.625789 107.804511) (end 136.694211 107.804511) (width 0.25) (layer "B.Cu") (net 28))
 (segment (start 139.51452 90.10148) (end 139.51452 105.91578) (width 0.25) (layer "B.Cu") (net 28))
 (segment (start 120.795489 78.274211) (end 121.4727 77.597) (width 0.25) (layer "F.Cu") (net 36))
 (segment (start 141.224 82.804) (end 141.224 82.981) (width 0.25) (layer "F.Cu") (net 36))
 (segment (start 116.84 71.12) (end 114.780001 73.179999) (width 0.25) (layer "F.Cu") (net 36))
 (segment (start 114.780001 82.522001) (end 117.756999 82.522001) (width 0.25) (layer "F.Cu") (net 36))
 (segment (start 121.4727 77.597) (end 136.017 77.597) (width 0.25) (layer "F.Cu") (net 36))
 (segment (start 117.756999 82.522001) (end 120.795489 79.483511) (width 0.25) (layer "F.Cu") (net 36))
 (segment (start 120.795489 79.483511) (end 120.795489 78.274211) (width 0.25) (layer "F.Cu") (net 36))
 (segment (start 114.780001 73.179999) (end 114.780001 82.522001) (width 0.25) (layer "F.Cu") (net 36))
 (segment (start 137.16 78.74) (end 141.224 82.804) (width 0.25) (layer "F.Cu") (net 36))
 (segment (start 136.017 77.597) (end 137.16 78.74) (width 0.25) (layer "F.Cu") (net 36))
 (segment (start 107.99 105.41) (end 107.99 108.45) (width 0.25) (layer "B.Cu") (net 3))
 (segment (start 108.331 103.93763) (end 108.331 87.376) (width 0.25) (layer "B.Cu") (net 3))
 (segment (start 108.331 87.376) (end 110.363 87.376) (width 0.25) (layer "B.Cu") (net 3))
 (segment (start 107.99 108.45) (end 107.22 109.22) (width 0.25) (layer "B.Cu") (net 3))
 (segment (start 107.99 105.41) (end 107.99 104.27863) (width 0.25) (layer "B.Cu") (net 3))
 (segment (start 107.99 104.27863) (end 108.331 103.93763) (width 0.25) (layer "B.Cu") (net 3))
 (segment (start 110.49 105.41) (end 110.49 107.95) (width 0.25) (layer "B.Cu") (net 4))
 (segment (start 110.363 94.996) (end 109.238489 96.120511) (width 0.25) (layer "B.Cu") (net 4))
 (segment (start 110.49 107.95) (end 109.22 109.22) (width 0.25) (layer "B.Cu") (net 4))
 (segment (start 109.897211 98.660511) (end 110.537811 98.660511) (width 0.25) (layer "B.Cu") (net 4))
 (segment (start 111.506 104.394) (end 110.49 105.41) (width 0.25) (layer "B.Cu") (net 4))
 (segment (start 110.537811 98.660511) (end 111.506 99.6287) (width 0.25) (layer "B.Cu") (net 4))
 (segment (start 109.238489 98.001789) (end 109.897211 98.660511) (width 0.25) (layer "B.Cu") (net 4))
 (segment (start 109.238489 96.120511) (end 109.238489 98.001789) (width 0.25) (layer "B.Cu") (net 4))
 (segment (start 111.506 99.6287) (end 111.506 104.394) (width 0.25) (layer "B.Cu") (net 4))
 (segment (start 139.065 102.235) (end 137.16 104.14) (width 0.25) (layer "B.Cu") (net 8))
 (segment (start 120.833489 53.881511) (end 121.92 52.795) (width 0.25) (layer "B.Cu") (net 8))
 (segment (start 115.663489 53.881511) (end 120.833489 53.881511) (width 0.25) (layer "B.Cu") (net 8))
 (segment (start 139.065 69.94) (end 139.065 102.235) (width 0.25) (layer "B.Cu") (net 8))
 (segment (start 121.92 52.795) (end 139.065 69.94) (width 0.25) (layer "B.Cu") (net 8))
 (segment (start 114.935 54.61) (end 115.663489 53.881511) (width 0.25) (layer "B.Cu") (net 8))
 (segment (start 117.517211 95.461789) (end 117.983 94.996) (width 0.25) (layer "B.Cu") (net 5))
 (segment (start 119.107511 97.070211) (end 118.448789 96.411489) (width 0.25) (layer "B.Cu") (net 5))
 (segment (start 114.34 105.41) (end 114.34 108.302468) (width 0.25) (layer "B.Cu") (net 5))
 (segment (start 119.107511 108.534957) (end 119.107511 97.070211) (width 0.25) (layer "B.Cu") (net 5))
 (segment (start 114.34 108.72) (end 114.84 109.22) (width 0.25) (layer "B.Cu") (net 5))
 (segment (start 114.34 105.41) (end 114.34 108.72) (width 0.25) (layer "B.Cu") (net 5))
 (segment (start 118.448789 96.411489) (end 117.517211 96.411489) (width 0.25) (layer "B.Cu") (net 5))
 (segment (start 117.222948 110.41952) (end 119.107511 108.534957) (width 0.25) (layer "B.Cu") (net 5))
 (segment (start 117.517211 96.411489) (end 117.517211 95.461789) (width 0.25) (layer "B.Cu") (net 5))
 (segment (start 114.34 108.302468) (end 116.457052 110.41952) (width 0.25) (layer "B.Cu") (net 5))
 (segment (start 116.457052 110.41952) (end 117.222948 110.41952) (width 0.25) (layer "B.Cu") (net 5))
 (segment (start 116.84 105.41) (end 116.84 109.22) (width 0.25) (layer "B.Cu") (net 6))
 (segment (start 117.983 87.376) (end 116.84 88.519) (width 0.25) (layer "B.Cu") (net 6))
 (segment (start 116.84 88.519) (end 116.84 105.41) (width 0.25) (layer "B.Cu") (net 6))
 (segment (start 104.21048 58.34952) (end 107.315 55.245) (width 0.25) (layer "B.Cu") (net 1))
 (segment (start 105.41 63.5) (end 104.21048 62.30048) (width 0.25) (layer "B.Cu") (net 1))
 (segment (start 104.21048 62.30048) (end 104.21048 58.34952) (width 0.25) (layer "B.Cu") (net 1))
 (segment (start 110.24601 51.435) (end 108.585 51.435) (width 0.25) (layer "B.Cu") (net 7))
 (segment (start 108.585 51.435) (end 107.315 52.705) (width 0.25) (layer "B.Cu") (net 7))
 (segment (start 111.83048 53.01947) (end 110.24601 51.435) (width 0.25) (layer "B.Cu") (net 7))
 (segment (start 111.83048 62.30048) (end 111.83048 53.01947) (width 0.25) (layer "B.Cu") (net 7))
 (segment (start 113.03 63.5) (end 111.83048 62.30048) (width 0.25) (layer "B.Cu") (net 7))
 (segment (start 118.16452 70.422013) (end 118.16452 74.87548) (width 0.25) (layer "B.Cu") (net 16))
 (segment (start 118.16452 74.87548) (end 116.84 76.2) (width 0.25) (layer "B.Cu") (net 16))
 (segment (start 109.855 62.112493) (end 118.16452 70.422013) (width 0.25) (layer "B.Cu") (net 16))
 (segment (start 109.855 55.245) (end 109.855 62.112493) (width 0.25) (layer "B.Cu") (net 16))
 (segment (start 111.487511 87.841789) (end 110.537811 88.791489) (width 0.25) (layer "B.Cu") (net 15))
 (segment (start 108.788969 98.501969) (end 110.363 100.076) (width 0.25) (layer "B.Cu") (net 15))
 (segment (start 110.828789 86.251489) (end 111.487511 86.910211) (width 0.25) (layer "B.Cu") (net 15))
 (segment (start 111.487511 86.910211) (end 111.487511 87.841789) (width 0.25) (layer "B.Cu") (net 15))
 (segment (start 108.788969 89.899731) (end 108.788969 98.501969) (width 0.25) (layer "B.Cu") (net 15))
 (segment (start 108.680489 85.566489) (end 109.347 86.233) (width 0.25) (layer "B.Cu") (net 15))
 (segment (start 109.855 52.705) (end 108.680489 53.879511) (width 0.25) (layer "B.Cu") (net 15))
 (segment (start 108.680489 53.879511) (end 108.680489 85.566489) (width 0.25) (layer "B.Cu") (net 15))
 (segment (start 109.35548 86.251489) (end 110.828789 86.251489) (width 0.25) (layer "B.Cu") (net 15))
 (segment (start 109.897211 88.791489) (end 108.788969 89.899731) (width 0.25) (layer "B.Cu") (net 15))
 (segment (start 110.537811 88.791489) (end 109.897211 88.791489) (width 0.25) (layer "B.Cu") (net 15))
 (segment (start 125.857 100.203) (end 121.92 104.14) (width 0.25) (layer "B.Cu") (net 12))
 (segment (start 125.857 61.812) (end 125.857 100.203) (width 0.25) (layer "B.Cu") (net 12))
 (segment (start 121.92 57.875) (end 125.857 61.812) (width 0.25) (layer "B.Cu") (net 12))
 (segment (start 112.532532 60.415) (end 109.093 63.854532) (width 0.25) (layer "F.Cu") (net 13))
 (segment (start 112.794489 104.285489) (end 119.525489 104.285489) (width 0.25) (layer "F.Cu") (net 13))
 (segment (start 109.093 100.584) (end 112.794489 104.285489) (width 0.25) (layer "F.Cu") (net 13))
 (segment (start 109.093 63.854532) (end 109.093 100.584) (width 0.25) (layer "F.Cu") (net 13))
 (segment (start 119.38 60.415) (end 112.532532 60.415) (width 0.25) (layer "F.Cu") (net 13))
 (segment (start 119.525489 104.285489) (end 121.92 106.68) (width 0.25) (layer "F.Cu") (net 13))
 (segment (start 136.035489 105.555489) (end 137.16 106.68) (width 0.25) (layer "B.Cu") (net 11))
 (segment (start 121.469951 53.881511) (end 122.370793 53.881511) (width 0.25) (layer "B.Cu") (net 11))
 (segment (start 136.035489 103.674211) (end 136.035489 105.555489) (width 0.25) (layer "B.Cu") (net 11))
 (segment (start 138.43 102.211278) (end 137.625789 103.015489) (width 0.25) (layer "B.Cu") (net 11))
 (segment (start 120.466511 55.785049) (end 120.466511 54.884951) (width 0.25) (layer "B.Cu") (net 11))
 (segment (start 136.694211 103.015489) (end 136.035489 103.674211) (width 0.25) (layer "B.Cu") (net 11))
 (segment (start 138.43 69.940718) (end 138.43 102.211278) (width 0.25) (layer "B.Cu") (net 11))
 (segment (start 119.38 56.87156) (end 120.466511 55.785049) (width 0.25) (layer "B.Cu") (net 11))
 (segment (start 119.38 57.875) (end 119.38 56.87156) (width 0.25) (layer "B.Cu") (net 11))
 (segment (start 122.370793 53.881511) (end 138.43 69.940718) (width 0.25) (layer "B.Cu") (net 11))
 (segment (start 137.625789 103.015489) (end 136.694211 103.015489) (width 0.25) (layer "B.Cu") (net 11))
 (segment (start 120.466511 54.884951) (end 121.469951 53.881511) (width 0.25) (layer "B.Cu") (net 11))
 (segment (start 139.860489 97.644511) (end 125.875489 97.644511) (width 0.25) (layer "F.Cu") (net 26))
 (segment (start 125.875489 97.644511) (end 121.92 101.6) (width 0.25) (layer "F.Cu") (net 26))
 (segment (start 141.605 95.9) (end 139.860489 97.644511) (width 0.25) (layer "F.Cu") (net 26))
 (segment (start 140.430489 99.614511) (end 140.430489 106.902489) (width 0.25) (layer "B.Cu") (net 40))
 (segment (start 141.605 98.44) (end 140.430489 99.614511) (width 0.25) (layer "B.Cu") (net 40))
 (segment (start 140.430489 106.902489) (end 141.351 107.823) (width 0.25) (layer "B.Cu") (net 40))
 (segment (start 142.779511 99.805489) (end 142.779511 92.487511) (width 0.25) (layer "B.Cu") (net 38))
 (segment (start 141.605 100.98) (end 142.779511 99.805489) (width 0.25) (layer "B.Cu") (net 38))
 (segment (start 142.525511 101.900511) (end 141.605 100.98) (width 0.25) (layer "B.Cu") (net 38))
 (segment (start 136.508014 108.254031) (end 135.128 106.874017) (width 0.25) (layer "B.Cu") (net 38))
 (segment (start 137.811986 108.254031) (end 136.508014 108.254031) (width 0.25) (layer "B.Cu") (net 38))
 (segment (start 139.980969 106.085048) (end 137.811986 108.254031) (width 0.25) (layer "B.Cu") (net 38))
 (segment (start 141.224 90.932) (end 139.980969 92.175031) (width 0.25) (layer "B.Cu") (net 38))
 (segment (start 135.128 106.874017) (end 135.128 75.692) (width 0.25) (layer "B.Cu") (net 38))
 (segment (start 142.525511 109.188489) (end 142.525511 101.900511) (width 0.25) (layer "B.Cu") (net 38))
 (segment (start 139.980969 92.175031) (end 139.980969 106.085048) (width 0.25) (layer "B.Cu") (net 38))
 (segment (start 135.128 75.692) (end 137.16 73.66) (width 0.25) (layer "B.Cu") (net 38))
 (segment (start 141.351 110.363) (end 142.525511 109.188489) (width 0.25) (layer "B.Cu") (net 38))
 (segment (start 142.779511 92.487511) (end 141.224 90.932) (width 0.25) (layer "B.Cu") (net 38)))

